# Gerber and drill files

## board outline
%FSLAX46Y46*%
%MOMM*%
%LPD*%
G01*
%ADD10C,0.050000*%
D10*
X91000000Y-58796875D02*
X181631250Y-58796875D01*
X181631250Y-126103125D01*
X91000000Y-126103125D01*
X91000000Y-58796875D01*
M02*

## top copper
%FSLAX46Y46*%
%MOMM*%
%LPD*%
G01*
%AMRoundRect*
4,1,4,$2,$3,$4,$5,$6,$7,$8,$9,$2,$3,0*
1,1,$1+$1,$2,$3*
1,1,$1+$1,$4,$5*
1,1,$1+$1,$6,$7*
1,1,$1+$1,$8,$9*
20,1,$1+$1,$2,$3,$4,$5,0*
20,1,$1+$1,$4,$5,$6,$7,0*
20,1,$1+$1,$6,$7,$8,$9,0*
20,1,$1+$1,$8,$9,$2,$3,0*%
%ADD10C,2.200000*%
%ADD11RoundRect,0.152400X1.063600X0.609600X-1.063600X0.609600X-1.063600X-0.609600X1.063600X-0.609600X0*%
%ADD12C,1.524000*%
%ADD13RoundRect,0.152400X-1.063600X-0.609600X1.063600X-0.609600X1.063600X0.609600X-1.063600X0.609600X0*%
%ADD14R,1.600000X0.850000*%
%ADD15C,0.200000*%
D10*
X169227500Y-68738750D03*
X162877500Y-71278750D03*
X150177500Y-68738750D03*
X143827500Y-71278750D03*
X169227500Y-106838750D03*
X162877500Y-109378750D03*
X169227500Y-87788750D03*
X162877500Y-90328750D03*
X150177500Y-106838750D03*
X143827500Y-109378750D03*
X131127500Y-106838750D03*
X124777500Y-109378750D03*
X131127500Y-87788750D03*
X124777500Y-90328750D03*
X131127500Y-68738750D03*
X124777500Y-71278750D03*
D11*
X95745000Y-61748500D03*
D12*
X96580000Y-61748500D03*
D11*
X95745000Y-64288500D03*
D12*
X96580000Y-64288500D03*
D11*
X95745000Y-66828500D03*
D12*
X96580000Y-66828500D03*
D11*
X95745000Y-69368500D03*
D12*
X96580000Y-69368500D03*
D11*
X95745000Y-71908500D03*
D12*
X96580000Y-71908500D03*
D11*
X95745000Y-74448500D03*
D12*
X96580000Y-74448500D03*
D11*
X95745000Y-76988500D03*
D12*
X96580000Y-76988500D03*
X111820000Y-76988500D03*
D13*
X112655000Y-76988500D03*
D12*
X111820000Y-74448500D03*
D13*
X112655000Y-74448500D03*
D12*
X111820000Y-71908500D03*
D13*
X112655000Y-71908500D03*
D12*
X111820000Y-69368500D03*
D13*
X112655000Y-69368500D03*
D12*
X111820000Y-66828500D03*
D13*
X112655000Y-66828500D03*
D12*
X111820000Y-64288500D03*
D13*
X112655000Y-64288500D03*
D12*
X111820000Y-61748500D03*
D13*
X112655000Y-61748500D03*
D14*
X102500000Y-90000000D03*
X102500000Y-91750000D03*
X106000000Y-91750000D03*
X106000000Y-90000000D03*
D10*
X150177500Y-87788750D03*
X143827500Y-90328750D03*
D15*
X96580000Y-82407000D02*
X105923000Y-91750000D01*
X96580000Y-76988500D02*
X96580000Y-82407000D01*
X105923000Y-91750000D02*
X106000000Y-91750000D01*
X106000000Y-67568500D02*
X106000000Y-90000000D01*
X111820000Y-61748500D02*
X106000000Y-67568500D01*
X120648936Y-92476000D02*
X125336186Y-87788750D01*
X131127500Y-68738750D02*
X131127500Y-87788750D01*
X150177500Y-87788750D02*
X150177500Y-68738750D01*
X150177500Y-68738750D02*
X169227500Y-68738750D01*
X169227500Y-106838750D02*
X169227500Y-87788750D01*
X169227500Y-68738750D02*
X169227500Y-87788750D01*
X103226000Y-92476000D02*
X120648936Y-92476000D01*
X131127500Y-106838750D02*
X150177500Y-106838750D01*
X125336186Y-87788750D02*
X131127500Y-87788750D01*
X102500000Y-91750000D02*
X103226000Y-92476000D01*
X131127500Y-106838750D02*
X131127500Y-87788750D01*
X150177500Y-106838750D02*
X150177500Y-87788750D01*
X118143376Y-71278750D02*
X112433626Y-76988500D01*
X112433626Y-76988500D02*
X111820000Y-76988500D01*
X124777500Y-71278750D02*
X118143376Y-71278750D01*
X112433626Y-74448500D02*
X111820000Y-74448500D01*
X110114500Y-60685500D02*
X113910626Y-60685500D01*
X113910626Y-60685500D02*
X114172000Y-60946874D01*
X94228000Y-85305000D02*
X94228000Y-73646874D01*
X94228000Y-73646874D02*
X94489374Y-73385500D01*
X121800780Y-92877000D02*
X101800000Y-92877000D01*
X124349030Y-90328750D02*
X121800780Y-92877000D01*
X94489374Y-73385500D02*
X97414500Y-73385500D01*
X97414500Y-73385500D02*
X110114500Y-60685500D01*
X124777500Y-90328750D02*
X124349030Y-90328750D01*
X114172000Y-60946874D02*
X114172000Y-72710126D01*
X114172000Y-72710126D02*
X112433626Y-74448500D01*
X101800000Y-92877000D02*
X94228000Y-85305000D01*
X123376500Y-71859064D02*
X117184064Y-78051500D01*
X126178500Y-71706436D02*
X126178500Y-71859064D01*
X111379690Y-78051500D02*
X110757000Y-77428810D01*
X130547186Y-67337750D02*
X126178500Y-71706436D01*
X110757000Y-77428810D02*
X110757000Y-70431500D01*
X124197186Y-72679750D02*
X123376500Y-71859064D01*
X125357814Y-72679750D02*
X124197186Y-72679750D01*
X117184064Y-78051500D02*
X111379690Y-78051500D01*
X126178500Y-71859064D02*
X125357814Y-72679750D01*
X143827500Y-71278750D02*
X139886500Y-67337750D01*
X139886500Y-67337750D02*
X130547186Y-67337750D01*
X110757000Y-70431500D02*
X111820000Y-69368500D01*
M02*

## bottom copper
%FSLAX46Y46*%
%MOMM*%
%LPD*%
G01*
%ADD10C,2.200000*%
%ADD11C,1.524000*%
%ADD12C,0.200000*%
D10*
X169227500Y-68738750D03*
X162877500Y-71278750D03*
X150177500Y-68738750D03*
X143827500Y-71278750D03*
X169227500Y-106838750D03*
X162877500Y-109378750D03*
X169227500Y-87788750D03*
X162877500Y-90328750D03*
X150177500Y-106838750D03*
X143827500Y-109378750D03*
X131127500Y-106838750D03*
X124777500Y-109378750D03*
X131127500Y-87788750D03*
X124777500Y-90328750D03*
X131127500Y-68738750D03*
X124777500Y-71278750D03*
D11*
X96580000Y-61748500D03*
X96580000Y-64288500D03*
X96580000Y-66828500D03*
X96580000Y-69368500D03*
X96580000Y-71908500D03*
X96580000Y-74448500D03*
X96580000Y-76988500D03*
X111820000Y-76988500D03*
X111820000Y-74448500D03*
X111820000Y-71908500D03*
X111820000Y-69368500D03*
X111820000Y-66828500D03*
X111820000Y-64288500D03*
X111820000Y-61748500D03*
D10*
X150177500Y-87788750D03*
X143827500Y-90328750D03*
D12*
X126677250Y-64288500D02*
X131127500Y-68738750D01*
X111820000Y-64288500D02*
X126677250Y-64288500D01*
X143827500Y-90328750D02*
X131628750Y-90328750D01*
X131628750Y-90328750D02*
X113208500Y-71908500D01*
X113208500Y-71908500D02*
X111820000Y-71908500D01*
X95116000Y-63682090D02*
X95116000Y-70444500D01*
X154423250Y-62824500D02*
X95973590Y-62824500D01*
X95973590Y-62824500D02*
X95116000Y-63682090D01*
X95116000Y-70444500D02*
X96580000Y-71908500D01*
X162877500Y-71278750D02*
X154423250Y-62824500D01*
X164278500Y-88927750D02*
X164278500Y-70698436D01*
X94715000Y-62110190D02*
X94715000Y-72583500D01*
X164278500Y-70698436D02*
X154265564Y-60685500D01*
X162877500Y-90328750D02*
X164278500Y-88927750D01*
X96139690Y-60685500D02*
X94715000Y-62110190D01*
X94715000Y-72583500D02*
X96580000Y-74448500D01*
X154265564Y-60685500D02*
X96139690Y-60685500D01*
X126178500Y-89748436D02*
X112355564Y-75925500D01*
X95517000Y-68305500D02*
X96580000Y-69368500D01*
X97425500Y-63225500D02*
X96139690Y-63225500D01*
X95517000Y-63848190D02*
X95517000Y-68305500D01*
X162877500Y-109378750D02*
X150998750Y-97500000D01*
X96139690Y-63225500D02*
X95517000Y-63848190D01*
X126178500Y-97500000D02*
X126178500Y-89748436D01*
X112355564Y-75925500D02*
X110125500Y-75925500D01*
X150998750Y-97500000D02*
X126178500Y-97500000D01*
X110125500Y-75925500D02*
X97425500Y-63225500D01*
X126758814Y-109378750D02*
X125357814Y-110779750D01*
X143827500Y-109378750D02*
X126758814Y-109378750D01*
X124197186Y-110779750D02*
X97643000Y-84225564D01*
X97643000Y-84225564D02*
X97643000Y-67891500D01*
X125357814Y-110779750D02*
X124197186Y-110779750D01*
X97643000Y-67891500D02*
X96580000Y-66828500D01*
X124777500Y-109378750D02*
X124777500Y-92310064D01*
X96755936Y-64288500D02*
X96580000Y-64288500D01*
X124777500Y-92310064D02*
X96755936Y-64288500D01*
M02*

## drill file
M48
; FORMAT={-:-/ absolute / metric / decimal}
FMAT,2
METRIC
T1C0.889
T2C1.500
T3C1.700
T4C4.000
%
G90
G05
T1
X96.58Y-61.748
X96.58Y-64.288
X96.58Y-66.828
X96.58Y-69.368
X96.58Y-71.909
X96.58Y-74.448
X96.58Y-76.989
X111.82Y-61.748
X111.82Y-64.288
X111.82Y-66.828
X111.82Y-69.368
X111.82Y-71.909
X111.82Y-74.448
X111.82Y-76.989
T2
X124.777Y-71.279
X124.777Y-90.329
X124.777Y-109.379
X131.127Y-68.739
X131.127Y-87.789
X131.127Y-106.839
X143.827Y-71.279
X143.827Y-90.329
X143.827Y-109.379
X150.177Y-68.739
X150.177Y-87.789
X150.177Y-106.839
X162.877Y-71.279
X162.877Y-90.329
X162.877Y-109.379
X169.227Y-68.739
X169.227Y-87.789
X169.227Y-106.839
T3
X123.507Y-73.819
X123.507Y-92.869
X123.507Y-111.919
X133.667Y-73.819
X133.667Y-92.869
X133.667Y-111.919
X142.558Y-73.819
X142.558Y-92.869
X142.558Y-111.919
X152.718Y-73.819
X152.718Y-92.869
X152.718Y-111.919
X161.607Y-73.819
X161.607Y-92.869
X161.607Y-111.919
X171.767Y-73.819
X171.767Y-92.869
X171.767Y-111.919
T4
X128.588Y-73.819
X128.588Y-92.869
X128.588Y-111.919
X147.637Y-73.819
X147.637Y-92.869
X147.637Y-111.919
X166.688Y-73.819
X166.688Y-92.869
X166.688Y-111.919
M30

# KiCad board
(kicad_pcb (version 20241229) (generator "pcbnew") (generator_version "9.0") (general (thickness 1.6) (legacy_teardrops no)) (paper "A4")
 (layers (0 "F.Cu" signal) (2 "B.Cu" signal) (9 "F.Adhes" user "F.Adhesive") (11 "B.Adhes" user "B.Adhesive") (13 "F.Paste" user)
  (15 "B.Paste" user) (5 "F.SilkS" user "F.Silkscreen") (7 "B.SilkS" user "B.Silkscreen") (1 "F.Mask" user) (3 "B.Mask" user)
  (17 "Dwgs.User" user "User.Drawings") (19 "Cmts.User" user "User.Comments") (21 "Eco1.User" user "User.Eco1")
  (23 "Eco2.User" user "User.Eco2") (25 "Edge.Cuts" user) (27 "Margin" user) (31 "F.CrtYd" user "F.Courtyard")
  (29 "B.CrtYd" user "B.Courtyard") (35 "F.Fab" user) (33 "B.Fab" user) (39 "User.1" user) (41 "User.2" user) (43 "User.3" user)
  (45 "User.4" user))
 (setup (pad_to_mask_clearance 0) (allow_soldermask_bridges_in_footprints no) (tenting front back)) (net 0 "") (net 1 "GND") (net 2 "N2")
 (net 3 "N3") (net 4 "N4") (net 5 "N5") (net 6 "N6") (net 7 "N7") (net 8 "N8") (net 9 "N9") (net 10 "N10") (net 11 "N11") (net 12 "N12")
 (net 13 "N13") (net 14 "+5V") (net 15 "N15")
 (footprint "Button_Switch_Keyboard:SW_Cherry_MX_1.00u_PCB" (layer "F.Cu") (at 169.2275 68.73875)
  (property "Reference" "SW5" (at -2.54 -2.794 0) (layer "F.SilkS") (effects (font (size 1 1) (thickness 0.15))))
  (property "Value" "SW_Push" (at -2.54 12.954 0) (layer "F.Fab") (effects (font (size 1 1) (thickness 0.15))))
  (pad "" np_thru_hole circle (at -7.62 5.08) (size 1.7 1.7) (drill 1.7) (layers "*.Cu" "*.Mask"))
  (pad "" np_thru_hole circle (at -2.54 5.08) (size 4 4) (drill 4) (layers "*.Cu" "*.Mask"))
  (pad "" np_thru_hole circle (at 2.54 5.08) (size 1.7 1.7) (drill 1.7) (layers "*.Cu" "*.Mask"))
  (pad "1" thru_hole circle (at 0 0) (size 2.2 2.2) (drill 1.5) (layers "*.Cu" "*.Mask") (remove_unused_layers no) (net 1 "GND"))
  (pad "2" thru_hole circle (at -6.35 2.54) (size 2.2 2.2) (drill 1.5) (layers "*.Cu" "*.Mask") (remove_unused_layers no) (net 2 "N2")))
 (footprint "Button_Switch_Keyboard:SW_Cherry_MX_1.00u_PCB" (layer "F.Cu") (at 150.1775 68.73875)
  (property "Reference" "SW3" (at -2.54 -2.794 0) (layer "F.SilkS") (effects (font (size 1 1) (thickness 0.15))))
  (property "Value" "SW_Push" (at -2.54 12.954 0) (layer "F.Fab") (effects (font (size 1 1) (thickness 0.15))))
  (pad "" np_thru_hole circle (at -7.62 5.08) (size 1.7 1.7) (drill 1.7) (layers "*.Cu" "*.Mask"))
  (pad "" np_thru_hole circle (at -2.54 5.08) (size 4 4) (drill 4) (layers "*.Cu" "*.Mask"))
  (pad "" np_thru_hole circle (at 2.54 5.08) (size 1.7 1.7) (drill 1.7) (layers "*.Cu" "*.Mask"))
  (pad "1" thru_hole circle (at 0 0) (size 2.2 2.2) (drill 1.5) (layers "*.Cu" "*.Mask") (remove_unused_layers no) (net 1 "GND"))
  (pad "2" thru_hole circle (at -6.35 2.54) (size 2.2 2.2) (drill 1.5) (layers "*.Cu" "*.Mask") (remove_unused_layers no) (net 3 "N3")))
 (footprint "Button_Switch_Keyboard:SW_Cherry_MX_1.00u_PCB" (layer "F.Cu") (at 169.2275 106.83875)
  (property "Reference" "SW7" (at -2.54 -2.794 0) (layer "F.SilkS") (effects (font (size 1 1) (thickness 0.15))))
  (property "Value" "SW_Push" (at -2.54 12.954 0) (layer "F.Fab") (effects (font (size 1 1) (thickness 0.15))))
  (pad "" np_thru_hole circle (at -7.62 5.08) (size 1.7 1.7) (drill 1.7) (layers "*.Cu" "*.Mask"))
  (pad "" np_thru_hole circle (at -2.54 5.08) (size 4 4) (drill 4) (layers "*.Cu" "*.Mask"))
  (pad "" np_thru_hole circle (at 2.54 5.08) (size 1.7 1.7) (drill 1.7) (layers "*.Cu" "*.Mask"))
  (pad "1" thru_hole circle (at 0 0) (size 2.2 2.2) (drill 1.5) (layers "*.Cu" "*.Mask") (remove_unused_layers no) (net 1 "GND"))
  (pad "2" thru_hole circle (at -6.35 2.54) (size 2.2 2.2) (drill 1.5) (layers "*.Cu" "*.Mask") (remove_unused_layers no) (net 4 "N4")))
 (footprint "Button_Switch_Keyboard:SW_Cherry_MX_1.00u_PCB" (layer "F.Cu") (at 169.2275 87.78875)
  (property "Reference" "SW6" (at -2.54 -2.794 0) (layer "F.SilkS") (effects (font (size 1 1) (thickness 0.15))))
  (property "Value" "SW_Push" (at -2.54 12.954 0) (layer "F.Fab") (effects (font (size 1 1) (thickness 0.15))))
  (pad "" np_thru_hole circle (at -7.62 5.08) (size 1.7 1.7) (drill 1.7) (layers "*.Cu" "*.Mask"))
  (pad "" np_thru_hole circle (at -2.54 5.08) (size 4 4) (drill 4) (layers "*.Cu" "*.Mask"))
  (pad "" np_thru_hole circle (at 2.54 5.08) (size 1.7 1.7) (drill 1.7) (layers "*.Cu" "*.Mask"))
  (pad "1" thru_hole circle (at 0 0) (size 2.2 2.2) (drill 1.5) (layers "*.Cu" "*.Mask") (remove_unused_layers no) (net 1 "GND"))
  (pad "2" thru_hole circle (at -6.35 2.54) (size 2.2 2.2) (drill 1.5) (layers "*.Cu" "*.Mask") (remove_unused_layers no) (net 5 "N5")))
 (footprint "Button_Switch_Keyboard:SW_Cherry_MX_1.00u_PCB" (layer "F.Cu") (at 150.1775 106.83875)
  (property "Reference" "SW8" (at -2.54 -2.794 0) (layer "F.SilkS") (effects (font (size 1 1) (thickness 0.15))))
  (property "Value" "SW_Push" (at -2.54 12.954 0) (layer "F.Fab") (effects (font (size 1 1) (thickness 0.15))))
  (pad "" np_thru_hole circle (at -7.62 5.08) (size 1.7 1.7) (drill 1.7) (layers "*.Cu" "*.Mask"))
  (pad "" np_thru_hole circle (at -2.54 5.08) (size 4 4) (drill 4) (layers "*.Cu" "*.Mask"))
  (pad "" np_thru_hole circle (at 2.54 5.08) (size 1.7 1.7) (drill 1.7) (layers "*.Cu" "*.Mask"))
  (pad "1" thru_hole circle (at 0 0) (size 2.2 2.2) (drill 1.5) (layers "*.Cu" "*.Mask") (remove_unused_layers no) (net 1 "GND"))
  (pad "2" thru_hole circle (at -6.35 2.54) (size 2.2 2.2) (drill 1.5) (layers "*.Cu" "*.Mask") (remove_unused_layers no) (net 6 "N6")))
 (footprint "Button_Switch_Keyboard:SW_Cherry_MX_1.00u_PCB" (layer "F.Cu") (at 131.1275 106.83875)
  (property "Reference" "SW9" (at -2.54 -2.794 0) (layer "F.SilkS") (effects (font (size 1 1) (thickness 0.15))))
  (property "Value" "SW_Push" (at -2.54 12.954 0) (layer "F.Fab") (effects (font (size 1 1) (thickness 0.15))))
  (pad "" np_thru_hole circle (at -7.62 5.08) (size 1.7 1.7) (drill 1.7) (layers "*.Cu" "*.Mask"))
  (pad "" np_thru_hole circle (at -2.54 5.08) (size 4 4) (drill 4) (layers "*.Cu" "*.Mask"))
  (pad "" np_thru_hole circle (at 2.54 5.08) (size 1.7 1.7) (drill 1.7) (layers "*.Cu" "*.Mask"))
  (pad "1" thru_hole circle (at 0 0) (size 2.2 2.2) (drill 1.5) (layers "*.Cu" "*.Mask") (remove_unused_layers no) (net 1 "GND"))
  (pad "2" thru_hole circle (at -6.35 2.54) (size 2.2 2.2) (drill 1.5) (layers "*.Cu" "*.Mask") (remove_unused_layers no) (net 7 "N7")))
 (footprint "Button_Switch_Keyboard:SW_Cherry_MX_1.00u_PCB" (layer "F.Cu") (at 131.1275 87.78875)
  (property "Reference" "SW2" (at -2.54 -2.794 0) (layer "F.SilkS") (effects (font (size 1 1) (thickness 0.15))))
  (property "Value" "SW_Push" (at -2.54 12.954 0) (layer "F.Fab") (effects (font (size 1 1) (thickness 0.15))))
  (pad "" np_thru_hole circle (at -7.62 5.08) (size 1.7 1.7) (drill 1.7) (layers "*.Cu" "*.Mask"))
  (pad "" np_thru_hole circle (at -2.54 5.08) (size 4 4) (drill 4) (layers "*.Cu" "*.Mask"))
  (pad "" np_thru_hole circle (at 2.54 5.08) (size 1.7 1.7) (drill 1.7) (layers "*.Cu" "*.Mask"))
  (pad "1" thru_hole circle (at 0 0) (size 2.2 2.2) (drill 1.5) (layers "*.Cu" "*.Mask") (remove_unused_layers no) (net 1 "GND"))
  (pad "2" thru_hole circle (at -6.35 2.54) (size 2.2 2.2) (drill 1.5) (layers "*.Cu" "*.Mask") (remove_unused_layers no) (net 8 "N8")))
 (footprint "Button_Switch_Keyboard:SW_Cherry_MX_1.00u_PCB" (layer "F.Cu") (at 131.1275 68.73875)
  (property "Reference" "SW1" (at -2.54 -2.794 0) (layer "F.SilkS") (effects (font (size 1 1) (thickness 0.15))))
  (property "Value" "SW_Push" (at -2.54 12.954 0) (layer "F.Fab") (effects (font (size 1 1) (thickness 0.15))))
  (pad "" np_thru_hole circle (at -7.62 5.08) (size 1.7 1.7) (drill 1.7) (layers "*.Cu" "*.Mask"))
  (pad "" np_thru_hole circle (at -2.54 5.08) (size 4 4) (drill 4) (layers "*.Cu" "*.Mask"))
  (pad "" np_thru_hole circle (at 2.54 5.08) (size 1.7 1.7) (drill 1.7) (layers "*.Cu" "*.Mask"))
  (pad "1" thru_hole circle (at 0 0) (size 2.2 2.2) (drill 1.5) (layers "*.Cu" "*.Mask") (remove_unused_layers no) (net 1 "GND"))
  (pad "2" thru_hole circle (at -6.35 2.54) (size 2.2 2.2) (drill 1.5) (layers "*.Cu" "*.Mask") (remove_unused_layers no) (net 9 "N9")))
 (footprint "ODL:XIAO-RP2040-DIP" (layer "F.Cu") (at 104.2 69.3685)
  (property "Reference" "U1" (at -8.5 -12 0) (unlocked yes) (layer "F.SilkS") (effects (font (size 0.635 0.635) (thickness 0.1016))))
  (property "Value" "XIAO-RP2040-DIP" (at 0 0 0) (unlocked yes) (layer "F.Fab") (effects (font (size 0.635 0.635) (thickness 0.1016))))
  (pad "1" smd roundrect (at -8.455 -7.62 180) (size 2.432 1.524) (layers "F.Cu" "F.Mask") (roundrect_rratio 0.1) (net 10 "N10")
   (thermal_bridge_angle 45))
  (pad "1" thru_hole circle (at -7.62 -7.62 180) (size 1.524 1.524) (drill 0.889) (layers "*.Cu" "*.Mask") (remove_unused_layers no)
   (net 10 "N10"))
  (pad "2" smd roundrect (at -8.455 -5.08 180) (size 2.432 1.524) (layers "F.Cu" "F.Mask") (roundrect_rratio 0.1) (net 7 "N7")
   (thermal_bridge_angle 45))
  (pad "2" thru_hole circle (at -7.62 -5.08 180) (size 1.524 1.524) (drill 0.889) (layers "*.Cu" "*.Mask") (remove_unused_layers no)
   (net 7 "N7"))
  (pad "3" smd roundrect (at -8.455 -2.54 180) (size 2.432 1.524) (layers "F.Cu" "F.Mask") (roundrect_rratio 0.1) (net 6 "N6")
   (thermal_bridge_angle 45))
  (pad "3" thru_hole circle (at -7.62 -2.54 180) (size 1.524 1.524) (drill 0.889) (layers "*.Cu" "*.Mask") (remove_unused_layers no)
   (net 6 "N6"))
  (pad "4" smd roundrect (at -8.455 0 180) (size 2.432 1.524) (layers "F.Cu" "F.Mask") (roundrect_rratio 0.1) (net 4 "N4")
   (thermal_bridge_angle 45))
  (pad "4" thru_hole circle (at -7.62 0 180) (size 1.524 1.524) (drill 0.889) (layers "*.Cu" "*.Mask") (remove_unused_layers no)
   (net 4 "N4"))
  (pad "5" smd roundrect (at -8.455 2.54 180) (size 2.432 1.524) (layers "F.Cu" "F.Mask") (roundrect_rratio 0.1) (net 2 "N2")
   (thermal_bridge_angle 45))
  (pad "5" thru_hole circle (at -7.62 2.54 180) (size 1.524 1.524) (drill 0.889) (layers "*.Cu" "*.Mask") (remove_unused_layers no)
   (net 2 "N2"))
  (pad "6" smd roundrect (at -8.455 5.08 180) (size 2.432 1.524) (layers "F.Cu" "F.Mask") (roundrect_rratio 0.1) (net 5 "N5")
   (thermal_bridge_angle 45))
  (pad "6" thru_hole circle (at -7.62 5.08 180) (size 1.524 1.524) (drill 0.889) (layers "*.Cu" "*.Mask") (remove_unused_layers no)
   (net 5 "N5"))
  (pad "7" smd roundrect (at -8.455 7.62 180) (size 2.432 1.524) (layers "F.Cu" "F.Mask") (roundrect_rratio 0.1) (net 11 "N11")
   (thermal_bridge_angle 45))
  (pad "7" thru_hole circle (at -7.62 7.62 180) (size 1.524 1.524) (drill 0.889) (layers "*.Cu" "*.Mask") (remove_unused_layers no)
   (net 11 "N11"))
  (pad "8" thru_hole circle (at 7.62 7.62) (size 1.524 1.524) (drill 0.889) (layers "*.Cu" "*.Mask") (remove_unused_layers no) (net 9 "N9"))
  (pad "8" smd roundrect (at 8.455 7.62) (size 2.432 1.524) (layers "F.Cu" "F.Mask") (roundrect_rratio 0.1) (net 9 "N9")
   (thermal_bridge_angle 45))
  (pad "9" thru_hole circle (at 7.62 5.08) (size 1.524 1.524) (drill 0.889) (layers "*.Cu" "*.Mask") (remove_unused_layers no) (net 8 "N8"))
  (pad "9" smd roundrect (at 8.455 5.08) (size 2.432 1.524) (layers "F.Cu" "F.Mask") (roundrect_rratio 0.1) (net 8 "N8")
   (thermal_bridge_angle 45))
  (pad "10" thru_hole circle (at 7.62 2.54) (size 1.524 1.524) (drill 0.889) (layers "*.Cu" "*.Mask") (remove_unused_layers no)
   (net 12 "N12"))
  (pad "10" smd roundrect (at 8.455 2.54) (size 2.432 1.524) (layers "F.Cu" "F.Mask") (roundrect_rratio 0.1) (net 12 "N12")
   (thermal_bridge_angle 45))
  (pad "11" thru_hole circle (at 7.62 0) (size 1.524 1.524) (drill 0.889) (layers "*.Cu" "*.Mask") (remove_unused_layers no) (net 3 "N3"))
  (pad "11" smd roundrect (at 8.455 0) (size 2.432 1.524) (layers "F.Cu" "F.Mask") (roundrect_rratio 0.1) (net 3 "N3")
   (thermal_bridge_angle 45))
  (pad "12" thru_hole circle (at 7.62 -2.54) (size 1.524 1.524) (drill 0.889) (layers "*.Cu" "*.Mask") (remove_unused_layers no)
   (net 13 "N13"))
  (pad "12" smd roundrect (at 8.455 -2.54) (size 2.432 1.524) (layers "F.Cu" "F.Mask") (roundrect_rratio 0.1) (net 13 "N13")
   (thermal_bridge_angle 45))
  (pad "13" thru_hole circle (at 7.62 -5.08) (size 1.524 1.524) (drill 0.889) (layers "*.Cu" "*.Mask") (remove_unused_layers no)
   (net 1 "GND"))
  (pad "13" smd roundrect (at 8.455 -5.08) (size 2.432 1.524) (layers "F.Cu" "F.Mask") (roundrect_rratio 0.1) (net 1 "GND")
   (thermal_bridge_angle 45))
  (pad "14" thru_hole circle (at 7.62 -7.62) (size 1.524 1.524) (drill 0.889) (layers "*.Cu" "*.Mask") (remove_unused_layers no)
   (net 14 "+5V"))
  (pad "14" smd roundrect (at 8.455 -7.62) (size 2.432 1.524) (layers "F.Cu" "F.Mask") (roundrect_rratio 0.1) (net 14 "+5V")
   (thermal_bridge_angle 45)))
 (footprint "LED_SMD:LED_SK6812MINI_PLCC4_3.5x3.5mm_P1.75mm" (layer "F.Cu") (at 104.25 90.875)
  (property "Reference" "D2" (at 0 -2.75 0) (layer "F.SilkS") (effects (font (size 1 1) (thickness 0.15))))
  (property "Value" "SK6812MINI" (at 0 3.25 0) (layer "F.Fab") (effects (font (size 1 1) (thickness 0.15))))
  (pad "1" smd rect (at -1.75 -0.875) (size 1.6 0.85) (layers "F.Cu" "F.Mask" "F.Paste") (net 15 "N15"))
  (pad "2" smd rect (at -1.75 0.875) (size 1.6 0.85) (layers "F.Cu" "F.Mask" "F.Paste") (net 1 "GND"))
  (pad "3" smd rect (at 1.75 0.875) (size 1.6 0.85) (layers "F.Cu" "F.Mask" "F.Paste") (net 11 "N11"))
  (pad "4" smd rect (at 1.75 -0.875) (size 1.6 0.85) (layers "F.Cu" "F.Mask" "F.Paste") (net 14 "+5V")))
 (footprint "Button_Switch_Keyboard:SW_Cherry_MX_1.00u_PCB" (layer "F.Cu") (at 150.1775 87.78875)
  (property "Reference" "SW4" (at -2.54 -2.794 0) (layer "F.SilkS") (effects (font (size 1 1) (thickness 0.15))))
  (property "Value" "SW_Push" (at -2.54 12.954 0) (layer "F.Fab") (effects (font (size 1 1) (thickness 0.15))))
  (pad "" np_thru_hole circle (at -7.62 5.08) (size 1.7 1.7) (drill 1.7) (layers "*.Cu" "*.Mask"))
  (pad "" np_thru_hole circle (at -2.54 5.08) (size 4 4) (drill 4) (layers "*.Cu" "*.Mask"))
  (pad "" np_thru_hole circle (at 2.54 5.08) (size 1.7 1.7) (drill 1.7) (layers "*.Cu" "*.Mask"))
  (pad "1" thru_hole circle (at 0 0) (size 2.2 2.2) (drill 1.5) (layers "*.Cu" "*.Mask") (remove_unused_layers no) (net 1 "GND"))
  (pad "2" thru_hole circle (at -6.35 2.54) (size 2.2 2.2) (drill 1.5) (layers "*.Cu" "*.Mask") (remove_unused_layers no) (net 12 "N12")))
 (gr_rect (start 91 58.796875) (end 181.63125 126.103125) (stroke (width 0.05) (type default)) (fill no) (layer "Edge.Cuts"))
 (segment (start 96.58 82.407) (end 105.923 91.75) (width 0.2) (layer "F.Cu") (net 11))
 (segment (start 96.58 76.9885) (end 96.58 82.407) (width 0.2) (layer "F.Cu") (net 11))
 (segment (start 105.923 91.75) (end 106 91.75) (width 0.2) (layer "F.Cu") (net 11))
 (segment (start 106 67.5685) (end 106 90) (width 0.2) (layer "F.Cu") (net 14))
 (segment (start 111.82 61.7485) (end 106 67.5685) (width 0.2) (layer "F.Cu") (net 14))
 (segment (start 120.648936 92.476) (end 125.336186 87.78875) (width 0.2) (layer "F.Cu") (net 1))
 (segment (start 131.1275 68.73875) (end 131.1275 87.78875) (width 0.2) (layer "F.Cu") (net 1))
 (segment (start 150.1775 87.78875) (end 150.1775 68.73875) (width 0.2) (layer "F.Cu") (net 1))
 (segment (start 150.1775 68.73875) (end 169.2275 68.73875) (width 0.2) (layer "F.Cu") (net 1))
 (segment (start 169.2275 106.83875) (end 169.2275 87.78875) (width 0.2) (layer "F.Cu") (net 1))
 (segment (start 169.2275 68.73875) (end 169.2275 87.78875) (width 0.2) (layer "F.Cu") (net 1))
 (segment (start 103.226 92.476) (end 120.648936 92.476) (width 0.2) (layer "F.Cu") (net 1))
 (segment (start 131.1275 106.83875) (end 150.1775 106.83875) (width 0.2) (layer "F.Cu") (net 1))
 (segment (start 125.336186 87.78875) (end 131.1275 87.78875) (width 0.2) (layer "F.Cu") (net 1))
 (segment (start 102.5 91.75) (end 103.226 92.476) (width 0.2) (layer "F.Cu") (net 1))
 (segment (start 131.1275 106.83875) (end 131.1275 87.78875) (width 0.2) (layer "F.Cu") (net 1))
 (segment (start 150.1775 106.83875) (end 150.1775 87.78875) (width 0.2) (layer "F.Cu") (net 1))
 (segment (start 126.67725 64.2885) (end 131.1275 68.73875) (width 0.2) (layer "B.Cu") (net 1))
 (segment (start 111.82 64.2885) (end 126.67725 64.2885) (width 0.2) (layer "B.Cu") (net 1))
 (segment (start 118.143376 71.27875) (end 112.433626 76.9885) (width 0.2) (layer "F.Cu") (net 9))
 (segment (start 112.433626 76.9885) (end 111.82 76.9885) (width 0.2) (layer "F.Cu") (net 9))
 (segment (start 124.7775 71.27875) (end 118.143376 71.27875) (width 0.2) (layer "F.Cu") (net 9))
 (segment (start 112.433626 74.4485) (end 111.82 74.4485) (width 0.2) (layer "F.Cu") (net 8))
 (segment (start 110.1145 60.6855) (end 113.910626 60.6855) (width 0.2) (layer "F.Cu") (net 8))
 (segment (start 113.910626 60.6855) (end 114.172 60.946874) (width 0.2) (layer "F.Cu") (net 8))
 (segment (start 94.228 85.305) (end 94.228 73.646874) (width 0.2) (layer "F.Cu") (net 8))
 (segment (start 94.228 73.646874) (end 94.489374 73.3855) (width 0.2) (layer "F.Cu") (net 8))
 (segment (start 121.80078 92.877) (end 101.8 92.877) (width 0.2) (layer "F.Cu") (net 8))
 (segment (start 124.34903 90.32875) (end 121.80078 92.877) (width 0.2) (layer "F.Cu") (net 8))
 (segment (start 94.489374 73.3855) (end 97.4145 73.3855) (width 0.2) (layer "F.Cu") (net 8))
 (segment (start 97.4145 73.3855) (end 110.1145 60.6855) (width 0.2) (layer "F.Cu") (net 8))
 (segment (start 124.7775 90.32875) (end 124.34903 90.32875) (width 0.2) (layer "F.Cu") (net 8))
 (segment (start 114.172 60.946874) (end 114.172 72.710126) (width 0.2) (layer "F.Cu") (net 8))
 (segment (start 114.172 72.710126) (end 112.433626 74.4485) (width 0.2) (layer "F.Cu") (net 8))
 (segment (start 101.8 92.877) (end 94.228 85.305) (width 0.2) (layer "F.Cu") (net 8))
 (segment (start 123.3765 71.859064) (end 117.184064 78.0515) (width 0.2) (layer "F.Cu") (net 3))
 (segment (start 126.1785 71.706436) (end 126.1785 71.859064) (width 0.2) (layer "F.Cu") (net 3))
 (segment (start 111.37969 78.0515) (end 110.757 77.42881) (width 0.2) (layer "F.Cu") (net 3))
 (segment (start 130.547186 67.33775) (end 126.1785 71.706436) (width 0.2) (layer "F.Cu") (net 3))
 (segment (start 110.757 77.42881) (end 110.757 70.4315) (width 0.2) (layer "F.Cu") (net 3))
 (segment (start 124.197186 72.67975) (end 123.3765 71.859064) (width 0.2) (layer "F.Cu") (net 3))
 (segment (start 125.357814 72.67975) (end 124.197186 72.67975) (width 0.2) (layer "F.Cu") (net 3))
 (segment (start 117.184064 78.0515) (end 111.37969 78.0515) (width 0.2) (layer "F.Cu") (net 3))
 (segment (start 126.1785 71.859064) (end 125.357814 72.67975) (width 0.2) (layer "F.Cu") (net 3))
 (segment (start 143.8275 71.27875) (end 139.8865 67.33775) (width 0.2) (layer "F.Cu") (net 3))
 (segment (start 139.8865 67.33775) (end 130.547186 67.33775) (width 0.2) (layer "F.Cu") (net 3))
 (segment (start 110.757 70.4315) (end 111.82 69.3685) (width 0.2) (layer "F.Cu") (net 3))
 (segment (start 143.8275 90.32875) (end 131.62875 90.32875) (width 0.2) (layer "B.Cu") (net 12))
 (segment (start 131.62875 90.32875) (end 113.2085 71.9085) (width 0.2) (layer "B.Cu") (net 12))
 (segment (start 113.2085 71.9085) (end 111.82 71.9085) (width 0.2) (layer "B.Cu") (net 12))
 (segment (start 95.116 63.68209) (end 95.116 70.4445) (width 0.2) (layer "B.Cu") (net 2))
 (segment (start 154.42325 62.8245) (end 95.97359 62.8245) (width 0.2) (layer "B.Cu") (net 2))
 (segment (start 95.97359 62.8245) (end 95.116 63.68209) (width 0.2) (layer "B.Cu") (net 2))
 (segment (start 95.116 70.4445) (end 96.58 71.9085) (width 0.2) (layer "B.Cu") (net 2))
 (segment (start 162.8775 71.27875) (end 154.42325 62.8245) (width 0.2) (layer "B.Cu") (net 2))
 (segment (start 164.2785 88.92775) (end 164.2785 70.698436) (width 0.2) (layer "B.Cu") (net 5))
 (segment (start 94.715 62.11019) (end 94.715 72.5835) (width 0.2) (layer "B.Cu") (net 5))
 (segment (start 164.2785 70.698436) (end 154.265564 60.6855) (width 0.2) (layer "B.Cu") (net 5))
 (segment (start 162.8775 90.32875) (end 164.2785 88.92775) (width 0.2) (layer "B.Cu") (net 5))
 (segment (start 96.13969 60.6855) (end 94.715 62.11019) (width 0.2) (layer "B.Cu") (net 5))
 (segment (start 94.715 72.5835) (end 96.58 74.4485) (width 0.2) (layer "B.Cu") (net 5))
 (segment (start 154.265564 60.6855) (end 96.13969 60.6855) (width 0.2) (layer "B.Cu") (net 5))
 (segment (start 126.1785 89.748436) (end 112.355564 75.9255) (width 0.2) (layer "B.Cu") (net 4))
 (segment (start 95.517 68.3055) (end 96.58 69.3685) (width 0.2) (layer "B.Cu") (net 4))
 (segment (start 97.4255 63.2255) (end 96.13969 63.2255) (width 0.2) (layer "B.Cu") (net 4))
 (segment (start 95.517 63.84819) (end 95.517 68.3055) (width 0.2) (layer "B.Cu") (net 4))
 (segment (start 162.8775 109.37875) (end 150.99875 97.5) (width 0.2) (layer "B.Cu") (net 4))
 (segment (start 96.13969 63.2255) (end 95.517 63.84819) (width 0.2) (layer "B.Cu") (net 4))
 (segment (start 126.1785 97.5) (end 126.1785 89.748436) (width 0.2) (layer "B.Cu") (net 4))
 (segment (start 112.355564 75.9255) (end 110.1255 75.9255) (width 0.2) (layer "B.Cu") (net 4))
 (segment (start 150.99875 97.5) (end 126.1785 97.5) (width 0.2) (layer "B.Cu") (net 4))
 (segment (start 110.1255 75.9255) (end 97.4255 63.2255) (width 0.2) (layer "B.Cu") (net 4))
 (segment (start 126.758814 109.37875) (end 125.357814 110.77975) (width 0.2) (layer "B.Cu") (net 6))
 (segment (start 143.8275 109.37875) (end 126.758814 109.37875) (width 0.2) (layer "B.Cu") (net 6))
 (segment (start 124.197186 110.77975) (end 97.643 84.225564) (width 0.2) (layer "B.Cu") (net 6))
 (segment (start 97.643 84.225564) (end 97.643 67.8915) (width 0.2) (layer "B.Cu") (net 6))
 (segment (start 125.357814 110.77975) (end 124.197186 110.77975) (width 0.2) (layer "B.Cu") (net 6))
 (segment (start 97.643 67.8915) (end 96.58 66.8285) (width 0.2) (layer "B.Cu") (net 6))
 (segment (start 124.7775 109.37875) (end 124.7775 92.310064) (width 0.2) (layer "B.Cu") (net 7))
 (segment (start 96.755936 64.2885) (end 96.58 64.2885) (width 0.2) (layer "B.Cu") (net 7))
 (segment (start 124.7775 92.310064) (end 96.755936 64.2885) (width 0.2) (layer "B.Cu") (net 7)))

